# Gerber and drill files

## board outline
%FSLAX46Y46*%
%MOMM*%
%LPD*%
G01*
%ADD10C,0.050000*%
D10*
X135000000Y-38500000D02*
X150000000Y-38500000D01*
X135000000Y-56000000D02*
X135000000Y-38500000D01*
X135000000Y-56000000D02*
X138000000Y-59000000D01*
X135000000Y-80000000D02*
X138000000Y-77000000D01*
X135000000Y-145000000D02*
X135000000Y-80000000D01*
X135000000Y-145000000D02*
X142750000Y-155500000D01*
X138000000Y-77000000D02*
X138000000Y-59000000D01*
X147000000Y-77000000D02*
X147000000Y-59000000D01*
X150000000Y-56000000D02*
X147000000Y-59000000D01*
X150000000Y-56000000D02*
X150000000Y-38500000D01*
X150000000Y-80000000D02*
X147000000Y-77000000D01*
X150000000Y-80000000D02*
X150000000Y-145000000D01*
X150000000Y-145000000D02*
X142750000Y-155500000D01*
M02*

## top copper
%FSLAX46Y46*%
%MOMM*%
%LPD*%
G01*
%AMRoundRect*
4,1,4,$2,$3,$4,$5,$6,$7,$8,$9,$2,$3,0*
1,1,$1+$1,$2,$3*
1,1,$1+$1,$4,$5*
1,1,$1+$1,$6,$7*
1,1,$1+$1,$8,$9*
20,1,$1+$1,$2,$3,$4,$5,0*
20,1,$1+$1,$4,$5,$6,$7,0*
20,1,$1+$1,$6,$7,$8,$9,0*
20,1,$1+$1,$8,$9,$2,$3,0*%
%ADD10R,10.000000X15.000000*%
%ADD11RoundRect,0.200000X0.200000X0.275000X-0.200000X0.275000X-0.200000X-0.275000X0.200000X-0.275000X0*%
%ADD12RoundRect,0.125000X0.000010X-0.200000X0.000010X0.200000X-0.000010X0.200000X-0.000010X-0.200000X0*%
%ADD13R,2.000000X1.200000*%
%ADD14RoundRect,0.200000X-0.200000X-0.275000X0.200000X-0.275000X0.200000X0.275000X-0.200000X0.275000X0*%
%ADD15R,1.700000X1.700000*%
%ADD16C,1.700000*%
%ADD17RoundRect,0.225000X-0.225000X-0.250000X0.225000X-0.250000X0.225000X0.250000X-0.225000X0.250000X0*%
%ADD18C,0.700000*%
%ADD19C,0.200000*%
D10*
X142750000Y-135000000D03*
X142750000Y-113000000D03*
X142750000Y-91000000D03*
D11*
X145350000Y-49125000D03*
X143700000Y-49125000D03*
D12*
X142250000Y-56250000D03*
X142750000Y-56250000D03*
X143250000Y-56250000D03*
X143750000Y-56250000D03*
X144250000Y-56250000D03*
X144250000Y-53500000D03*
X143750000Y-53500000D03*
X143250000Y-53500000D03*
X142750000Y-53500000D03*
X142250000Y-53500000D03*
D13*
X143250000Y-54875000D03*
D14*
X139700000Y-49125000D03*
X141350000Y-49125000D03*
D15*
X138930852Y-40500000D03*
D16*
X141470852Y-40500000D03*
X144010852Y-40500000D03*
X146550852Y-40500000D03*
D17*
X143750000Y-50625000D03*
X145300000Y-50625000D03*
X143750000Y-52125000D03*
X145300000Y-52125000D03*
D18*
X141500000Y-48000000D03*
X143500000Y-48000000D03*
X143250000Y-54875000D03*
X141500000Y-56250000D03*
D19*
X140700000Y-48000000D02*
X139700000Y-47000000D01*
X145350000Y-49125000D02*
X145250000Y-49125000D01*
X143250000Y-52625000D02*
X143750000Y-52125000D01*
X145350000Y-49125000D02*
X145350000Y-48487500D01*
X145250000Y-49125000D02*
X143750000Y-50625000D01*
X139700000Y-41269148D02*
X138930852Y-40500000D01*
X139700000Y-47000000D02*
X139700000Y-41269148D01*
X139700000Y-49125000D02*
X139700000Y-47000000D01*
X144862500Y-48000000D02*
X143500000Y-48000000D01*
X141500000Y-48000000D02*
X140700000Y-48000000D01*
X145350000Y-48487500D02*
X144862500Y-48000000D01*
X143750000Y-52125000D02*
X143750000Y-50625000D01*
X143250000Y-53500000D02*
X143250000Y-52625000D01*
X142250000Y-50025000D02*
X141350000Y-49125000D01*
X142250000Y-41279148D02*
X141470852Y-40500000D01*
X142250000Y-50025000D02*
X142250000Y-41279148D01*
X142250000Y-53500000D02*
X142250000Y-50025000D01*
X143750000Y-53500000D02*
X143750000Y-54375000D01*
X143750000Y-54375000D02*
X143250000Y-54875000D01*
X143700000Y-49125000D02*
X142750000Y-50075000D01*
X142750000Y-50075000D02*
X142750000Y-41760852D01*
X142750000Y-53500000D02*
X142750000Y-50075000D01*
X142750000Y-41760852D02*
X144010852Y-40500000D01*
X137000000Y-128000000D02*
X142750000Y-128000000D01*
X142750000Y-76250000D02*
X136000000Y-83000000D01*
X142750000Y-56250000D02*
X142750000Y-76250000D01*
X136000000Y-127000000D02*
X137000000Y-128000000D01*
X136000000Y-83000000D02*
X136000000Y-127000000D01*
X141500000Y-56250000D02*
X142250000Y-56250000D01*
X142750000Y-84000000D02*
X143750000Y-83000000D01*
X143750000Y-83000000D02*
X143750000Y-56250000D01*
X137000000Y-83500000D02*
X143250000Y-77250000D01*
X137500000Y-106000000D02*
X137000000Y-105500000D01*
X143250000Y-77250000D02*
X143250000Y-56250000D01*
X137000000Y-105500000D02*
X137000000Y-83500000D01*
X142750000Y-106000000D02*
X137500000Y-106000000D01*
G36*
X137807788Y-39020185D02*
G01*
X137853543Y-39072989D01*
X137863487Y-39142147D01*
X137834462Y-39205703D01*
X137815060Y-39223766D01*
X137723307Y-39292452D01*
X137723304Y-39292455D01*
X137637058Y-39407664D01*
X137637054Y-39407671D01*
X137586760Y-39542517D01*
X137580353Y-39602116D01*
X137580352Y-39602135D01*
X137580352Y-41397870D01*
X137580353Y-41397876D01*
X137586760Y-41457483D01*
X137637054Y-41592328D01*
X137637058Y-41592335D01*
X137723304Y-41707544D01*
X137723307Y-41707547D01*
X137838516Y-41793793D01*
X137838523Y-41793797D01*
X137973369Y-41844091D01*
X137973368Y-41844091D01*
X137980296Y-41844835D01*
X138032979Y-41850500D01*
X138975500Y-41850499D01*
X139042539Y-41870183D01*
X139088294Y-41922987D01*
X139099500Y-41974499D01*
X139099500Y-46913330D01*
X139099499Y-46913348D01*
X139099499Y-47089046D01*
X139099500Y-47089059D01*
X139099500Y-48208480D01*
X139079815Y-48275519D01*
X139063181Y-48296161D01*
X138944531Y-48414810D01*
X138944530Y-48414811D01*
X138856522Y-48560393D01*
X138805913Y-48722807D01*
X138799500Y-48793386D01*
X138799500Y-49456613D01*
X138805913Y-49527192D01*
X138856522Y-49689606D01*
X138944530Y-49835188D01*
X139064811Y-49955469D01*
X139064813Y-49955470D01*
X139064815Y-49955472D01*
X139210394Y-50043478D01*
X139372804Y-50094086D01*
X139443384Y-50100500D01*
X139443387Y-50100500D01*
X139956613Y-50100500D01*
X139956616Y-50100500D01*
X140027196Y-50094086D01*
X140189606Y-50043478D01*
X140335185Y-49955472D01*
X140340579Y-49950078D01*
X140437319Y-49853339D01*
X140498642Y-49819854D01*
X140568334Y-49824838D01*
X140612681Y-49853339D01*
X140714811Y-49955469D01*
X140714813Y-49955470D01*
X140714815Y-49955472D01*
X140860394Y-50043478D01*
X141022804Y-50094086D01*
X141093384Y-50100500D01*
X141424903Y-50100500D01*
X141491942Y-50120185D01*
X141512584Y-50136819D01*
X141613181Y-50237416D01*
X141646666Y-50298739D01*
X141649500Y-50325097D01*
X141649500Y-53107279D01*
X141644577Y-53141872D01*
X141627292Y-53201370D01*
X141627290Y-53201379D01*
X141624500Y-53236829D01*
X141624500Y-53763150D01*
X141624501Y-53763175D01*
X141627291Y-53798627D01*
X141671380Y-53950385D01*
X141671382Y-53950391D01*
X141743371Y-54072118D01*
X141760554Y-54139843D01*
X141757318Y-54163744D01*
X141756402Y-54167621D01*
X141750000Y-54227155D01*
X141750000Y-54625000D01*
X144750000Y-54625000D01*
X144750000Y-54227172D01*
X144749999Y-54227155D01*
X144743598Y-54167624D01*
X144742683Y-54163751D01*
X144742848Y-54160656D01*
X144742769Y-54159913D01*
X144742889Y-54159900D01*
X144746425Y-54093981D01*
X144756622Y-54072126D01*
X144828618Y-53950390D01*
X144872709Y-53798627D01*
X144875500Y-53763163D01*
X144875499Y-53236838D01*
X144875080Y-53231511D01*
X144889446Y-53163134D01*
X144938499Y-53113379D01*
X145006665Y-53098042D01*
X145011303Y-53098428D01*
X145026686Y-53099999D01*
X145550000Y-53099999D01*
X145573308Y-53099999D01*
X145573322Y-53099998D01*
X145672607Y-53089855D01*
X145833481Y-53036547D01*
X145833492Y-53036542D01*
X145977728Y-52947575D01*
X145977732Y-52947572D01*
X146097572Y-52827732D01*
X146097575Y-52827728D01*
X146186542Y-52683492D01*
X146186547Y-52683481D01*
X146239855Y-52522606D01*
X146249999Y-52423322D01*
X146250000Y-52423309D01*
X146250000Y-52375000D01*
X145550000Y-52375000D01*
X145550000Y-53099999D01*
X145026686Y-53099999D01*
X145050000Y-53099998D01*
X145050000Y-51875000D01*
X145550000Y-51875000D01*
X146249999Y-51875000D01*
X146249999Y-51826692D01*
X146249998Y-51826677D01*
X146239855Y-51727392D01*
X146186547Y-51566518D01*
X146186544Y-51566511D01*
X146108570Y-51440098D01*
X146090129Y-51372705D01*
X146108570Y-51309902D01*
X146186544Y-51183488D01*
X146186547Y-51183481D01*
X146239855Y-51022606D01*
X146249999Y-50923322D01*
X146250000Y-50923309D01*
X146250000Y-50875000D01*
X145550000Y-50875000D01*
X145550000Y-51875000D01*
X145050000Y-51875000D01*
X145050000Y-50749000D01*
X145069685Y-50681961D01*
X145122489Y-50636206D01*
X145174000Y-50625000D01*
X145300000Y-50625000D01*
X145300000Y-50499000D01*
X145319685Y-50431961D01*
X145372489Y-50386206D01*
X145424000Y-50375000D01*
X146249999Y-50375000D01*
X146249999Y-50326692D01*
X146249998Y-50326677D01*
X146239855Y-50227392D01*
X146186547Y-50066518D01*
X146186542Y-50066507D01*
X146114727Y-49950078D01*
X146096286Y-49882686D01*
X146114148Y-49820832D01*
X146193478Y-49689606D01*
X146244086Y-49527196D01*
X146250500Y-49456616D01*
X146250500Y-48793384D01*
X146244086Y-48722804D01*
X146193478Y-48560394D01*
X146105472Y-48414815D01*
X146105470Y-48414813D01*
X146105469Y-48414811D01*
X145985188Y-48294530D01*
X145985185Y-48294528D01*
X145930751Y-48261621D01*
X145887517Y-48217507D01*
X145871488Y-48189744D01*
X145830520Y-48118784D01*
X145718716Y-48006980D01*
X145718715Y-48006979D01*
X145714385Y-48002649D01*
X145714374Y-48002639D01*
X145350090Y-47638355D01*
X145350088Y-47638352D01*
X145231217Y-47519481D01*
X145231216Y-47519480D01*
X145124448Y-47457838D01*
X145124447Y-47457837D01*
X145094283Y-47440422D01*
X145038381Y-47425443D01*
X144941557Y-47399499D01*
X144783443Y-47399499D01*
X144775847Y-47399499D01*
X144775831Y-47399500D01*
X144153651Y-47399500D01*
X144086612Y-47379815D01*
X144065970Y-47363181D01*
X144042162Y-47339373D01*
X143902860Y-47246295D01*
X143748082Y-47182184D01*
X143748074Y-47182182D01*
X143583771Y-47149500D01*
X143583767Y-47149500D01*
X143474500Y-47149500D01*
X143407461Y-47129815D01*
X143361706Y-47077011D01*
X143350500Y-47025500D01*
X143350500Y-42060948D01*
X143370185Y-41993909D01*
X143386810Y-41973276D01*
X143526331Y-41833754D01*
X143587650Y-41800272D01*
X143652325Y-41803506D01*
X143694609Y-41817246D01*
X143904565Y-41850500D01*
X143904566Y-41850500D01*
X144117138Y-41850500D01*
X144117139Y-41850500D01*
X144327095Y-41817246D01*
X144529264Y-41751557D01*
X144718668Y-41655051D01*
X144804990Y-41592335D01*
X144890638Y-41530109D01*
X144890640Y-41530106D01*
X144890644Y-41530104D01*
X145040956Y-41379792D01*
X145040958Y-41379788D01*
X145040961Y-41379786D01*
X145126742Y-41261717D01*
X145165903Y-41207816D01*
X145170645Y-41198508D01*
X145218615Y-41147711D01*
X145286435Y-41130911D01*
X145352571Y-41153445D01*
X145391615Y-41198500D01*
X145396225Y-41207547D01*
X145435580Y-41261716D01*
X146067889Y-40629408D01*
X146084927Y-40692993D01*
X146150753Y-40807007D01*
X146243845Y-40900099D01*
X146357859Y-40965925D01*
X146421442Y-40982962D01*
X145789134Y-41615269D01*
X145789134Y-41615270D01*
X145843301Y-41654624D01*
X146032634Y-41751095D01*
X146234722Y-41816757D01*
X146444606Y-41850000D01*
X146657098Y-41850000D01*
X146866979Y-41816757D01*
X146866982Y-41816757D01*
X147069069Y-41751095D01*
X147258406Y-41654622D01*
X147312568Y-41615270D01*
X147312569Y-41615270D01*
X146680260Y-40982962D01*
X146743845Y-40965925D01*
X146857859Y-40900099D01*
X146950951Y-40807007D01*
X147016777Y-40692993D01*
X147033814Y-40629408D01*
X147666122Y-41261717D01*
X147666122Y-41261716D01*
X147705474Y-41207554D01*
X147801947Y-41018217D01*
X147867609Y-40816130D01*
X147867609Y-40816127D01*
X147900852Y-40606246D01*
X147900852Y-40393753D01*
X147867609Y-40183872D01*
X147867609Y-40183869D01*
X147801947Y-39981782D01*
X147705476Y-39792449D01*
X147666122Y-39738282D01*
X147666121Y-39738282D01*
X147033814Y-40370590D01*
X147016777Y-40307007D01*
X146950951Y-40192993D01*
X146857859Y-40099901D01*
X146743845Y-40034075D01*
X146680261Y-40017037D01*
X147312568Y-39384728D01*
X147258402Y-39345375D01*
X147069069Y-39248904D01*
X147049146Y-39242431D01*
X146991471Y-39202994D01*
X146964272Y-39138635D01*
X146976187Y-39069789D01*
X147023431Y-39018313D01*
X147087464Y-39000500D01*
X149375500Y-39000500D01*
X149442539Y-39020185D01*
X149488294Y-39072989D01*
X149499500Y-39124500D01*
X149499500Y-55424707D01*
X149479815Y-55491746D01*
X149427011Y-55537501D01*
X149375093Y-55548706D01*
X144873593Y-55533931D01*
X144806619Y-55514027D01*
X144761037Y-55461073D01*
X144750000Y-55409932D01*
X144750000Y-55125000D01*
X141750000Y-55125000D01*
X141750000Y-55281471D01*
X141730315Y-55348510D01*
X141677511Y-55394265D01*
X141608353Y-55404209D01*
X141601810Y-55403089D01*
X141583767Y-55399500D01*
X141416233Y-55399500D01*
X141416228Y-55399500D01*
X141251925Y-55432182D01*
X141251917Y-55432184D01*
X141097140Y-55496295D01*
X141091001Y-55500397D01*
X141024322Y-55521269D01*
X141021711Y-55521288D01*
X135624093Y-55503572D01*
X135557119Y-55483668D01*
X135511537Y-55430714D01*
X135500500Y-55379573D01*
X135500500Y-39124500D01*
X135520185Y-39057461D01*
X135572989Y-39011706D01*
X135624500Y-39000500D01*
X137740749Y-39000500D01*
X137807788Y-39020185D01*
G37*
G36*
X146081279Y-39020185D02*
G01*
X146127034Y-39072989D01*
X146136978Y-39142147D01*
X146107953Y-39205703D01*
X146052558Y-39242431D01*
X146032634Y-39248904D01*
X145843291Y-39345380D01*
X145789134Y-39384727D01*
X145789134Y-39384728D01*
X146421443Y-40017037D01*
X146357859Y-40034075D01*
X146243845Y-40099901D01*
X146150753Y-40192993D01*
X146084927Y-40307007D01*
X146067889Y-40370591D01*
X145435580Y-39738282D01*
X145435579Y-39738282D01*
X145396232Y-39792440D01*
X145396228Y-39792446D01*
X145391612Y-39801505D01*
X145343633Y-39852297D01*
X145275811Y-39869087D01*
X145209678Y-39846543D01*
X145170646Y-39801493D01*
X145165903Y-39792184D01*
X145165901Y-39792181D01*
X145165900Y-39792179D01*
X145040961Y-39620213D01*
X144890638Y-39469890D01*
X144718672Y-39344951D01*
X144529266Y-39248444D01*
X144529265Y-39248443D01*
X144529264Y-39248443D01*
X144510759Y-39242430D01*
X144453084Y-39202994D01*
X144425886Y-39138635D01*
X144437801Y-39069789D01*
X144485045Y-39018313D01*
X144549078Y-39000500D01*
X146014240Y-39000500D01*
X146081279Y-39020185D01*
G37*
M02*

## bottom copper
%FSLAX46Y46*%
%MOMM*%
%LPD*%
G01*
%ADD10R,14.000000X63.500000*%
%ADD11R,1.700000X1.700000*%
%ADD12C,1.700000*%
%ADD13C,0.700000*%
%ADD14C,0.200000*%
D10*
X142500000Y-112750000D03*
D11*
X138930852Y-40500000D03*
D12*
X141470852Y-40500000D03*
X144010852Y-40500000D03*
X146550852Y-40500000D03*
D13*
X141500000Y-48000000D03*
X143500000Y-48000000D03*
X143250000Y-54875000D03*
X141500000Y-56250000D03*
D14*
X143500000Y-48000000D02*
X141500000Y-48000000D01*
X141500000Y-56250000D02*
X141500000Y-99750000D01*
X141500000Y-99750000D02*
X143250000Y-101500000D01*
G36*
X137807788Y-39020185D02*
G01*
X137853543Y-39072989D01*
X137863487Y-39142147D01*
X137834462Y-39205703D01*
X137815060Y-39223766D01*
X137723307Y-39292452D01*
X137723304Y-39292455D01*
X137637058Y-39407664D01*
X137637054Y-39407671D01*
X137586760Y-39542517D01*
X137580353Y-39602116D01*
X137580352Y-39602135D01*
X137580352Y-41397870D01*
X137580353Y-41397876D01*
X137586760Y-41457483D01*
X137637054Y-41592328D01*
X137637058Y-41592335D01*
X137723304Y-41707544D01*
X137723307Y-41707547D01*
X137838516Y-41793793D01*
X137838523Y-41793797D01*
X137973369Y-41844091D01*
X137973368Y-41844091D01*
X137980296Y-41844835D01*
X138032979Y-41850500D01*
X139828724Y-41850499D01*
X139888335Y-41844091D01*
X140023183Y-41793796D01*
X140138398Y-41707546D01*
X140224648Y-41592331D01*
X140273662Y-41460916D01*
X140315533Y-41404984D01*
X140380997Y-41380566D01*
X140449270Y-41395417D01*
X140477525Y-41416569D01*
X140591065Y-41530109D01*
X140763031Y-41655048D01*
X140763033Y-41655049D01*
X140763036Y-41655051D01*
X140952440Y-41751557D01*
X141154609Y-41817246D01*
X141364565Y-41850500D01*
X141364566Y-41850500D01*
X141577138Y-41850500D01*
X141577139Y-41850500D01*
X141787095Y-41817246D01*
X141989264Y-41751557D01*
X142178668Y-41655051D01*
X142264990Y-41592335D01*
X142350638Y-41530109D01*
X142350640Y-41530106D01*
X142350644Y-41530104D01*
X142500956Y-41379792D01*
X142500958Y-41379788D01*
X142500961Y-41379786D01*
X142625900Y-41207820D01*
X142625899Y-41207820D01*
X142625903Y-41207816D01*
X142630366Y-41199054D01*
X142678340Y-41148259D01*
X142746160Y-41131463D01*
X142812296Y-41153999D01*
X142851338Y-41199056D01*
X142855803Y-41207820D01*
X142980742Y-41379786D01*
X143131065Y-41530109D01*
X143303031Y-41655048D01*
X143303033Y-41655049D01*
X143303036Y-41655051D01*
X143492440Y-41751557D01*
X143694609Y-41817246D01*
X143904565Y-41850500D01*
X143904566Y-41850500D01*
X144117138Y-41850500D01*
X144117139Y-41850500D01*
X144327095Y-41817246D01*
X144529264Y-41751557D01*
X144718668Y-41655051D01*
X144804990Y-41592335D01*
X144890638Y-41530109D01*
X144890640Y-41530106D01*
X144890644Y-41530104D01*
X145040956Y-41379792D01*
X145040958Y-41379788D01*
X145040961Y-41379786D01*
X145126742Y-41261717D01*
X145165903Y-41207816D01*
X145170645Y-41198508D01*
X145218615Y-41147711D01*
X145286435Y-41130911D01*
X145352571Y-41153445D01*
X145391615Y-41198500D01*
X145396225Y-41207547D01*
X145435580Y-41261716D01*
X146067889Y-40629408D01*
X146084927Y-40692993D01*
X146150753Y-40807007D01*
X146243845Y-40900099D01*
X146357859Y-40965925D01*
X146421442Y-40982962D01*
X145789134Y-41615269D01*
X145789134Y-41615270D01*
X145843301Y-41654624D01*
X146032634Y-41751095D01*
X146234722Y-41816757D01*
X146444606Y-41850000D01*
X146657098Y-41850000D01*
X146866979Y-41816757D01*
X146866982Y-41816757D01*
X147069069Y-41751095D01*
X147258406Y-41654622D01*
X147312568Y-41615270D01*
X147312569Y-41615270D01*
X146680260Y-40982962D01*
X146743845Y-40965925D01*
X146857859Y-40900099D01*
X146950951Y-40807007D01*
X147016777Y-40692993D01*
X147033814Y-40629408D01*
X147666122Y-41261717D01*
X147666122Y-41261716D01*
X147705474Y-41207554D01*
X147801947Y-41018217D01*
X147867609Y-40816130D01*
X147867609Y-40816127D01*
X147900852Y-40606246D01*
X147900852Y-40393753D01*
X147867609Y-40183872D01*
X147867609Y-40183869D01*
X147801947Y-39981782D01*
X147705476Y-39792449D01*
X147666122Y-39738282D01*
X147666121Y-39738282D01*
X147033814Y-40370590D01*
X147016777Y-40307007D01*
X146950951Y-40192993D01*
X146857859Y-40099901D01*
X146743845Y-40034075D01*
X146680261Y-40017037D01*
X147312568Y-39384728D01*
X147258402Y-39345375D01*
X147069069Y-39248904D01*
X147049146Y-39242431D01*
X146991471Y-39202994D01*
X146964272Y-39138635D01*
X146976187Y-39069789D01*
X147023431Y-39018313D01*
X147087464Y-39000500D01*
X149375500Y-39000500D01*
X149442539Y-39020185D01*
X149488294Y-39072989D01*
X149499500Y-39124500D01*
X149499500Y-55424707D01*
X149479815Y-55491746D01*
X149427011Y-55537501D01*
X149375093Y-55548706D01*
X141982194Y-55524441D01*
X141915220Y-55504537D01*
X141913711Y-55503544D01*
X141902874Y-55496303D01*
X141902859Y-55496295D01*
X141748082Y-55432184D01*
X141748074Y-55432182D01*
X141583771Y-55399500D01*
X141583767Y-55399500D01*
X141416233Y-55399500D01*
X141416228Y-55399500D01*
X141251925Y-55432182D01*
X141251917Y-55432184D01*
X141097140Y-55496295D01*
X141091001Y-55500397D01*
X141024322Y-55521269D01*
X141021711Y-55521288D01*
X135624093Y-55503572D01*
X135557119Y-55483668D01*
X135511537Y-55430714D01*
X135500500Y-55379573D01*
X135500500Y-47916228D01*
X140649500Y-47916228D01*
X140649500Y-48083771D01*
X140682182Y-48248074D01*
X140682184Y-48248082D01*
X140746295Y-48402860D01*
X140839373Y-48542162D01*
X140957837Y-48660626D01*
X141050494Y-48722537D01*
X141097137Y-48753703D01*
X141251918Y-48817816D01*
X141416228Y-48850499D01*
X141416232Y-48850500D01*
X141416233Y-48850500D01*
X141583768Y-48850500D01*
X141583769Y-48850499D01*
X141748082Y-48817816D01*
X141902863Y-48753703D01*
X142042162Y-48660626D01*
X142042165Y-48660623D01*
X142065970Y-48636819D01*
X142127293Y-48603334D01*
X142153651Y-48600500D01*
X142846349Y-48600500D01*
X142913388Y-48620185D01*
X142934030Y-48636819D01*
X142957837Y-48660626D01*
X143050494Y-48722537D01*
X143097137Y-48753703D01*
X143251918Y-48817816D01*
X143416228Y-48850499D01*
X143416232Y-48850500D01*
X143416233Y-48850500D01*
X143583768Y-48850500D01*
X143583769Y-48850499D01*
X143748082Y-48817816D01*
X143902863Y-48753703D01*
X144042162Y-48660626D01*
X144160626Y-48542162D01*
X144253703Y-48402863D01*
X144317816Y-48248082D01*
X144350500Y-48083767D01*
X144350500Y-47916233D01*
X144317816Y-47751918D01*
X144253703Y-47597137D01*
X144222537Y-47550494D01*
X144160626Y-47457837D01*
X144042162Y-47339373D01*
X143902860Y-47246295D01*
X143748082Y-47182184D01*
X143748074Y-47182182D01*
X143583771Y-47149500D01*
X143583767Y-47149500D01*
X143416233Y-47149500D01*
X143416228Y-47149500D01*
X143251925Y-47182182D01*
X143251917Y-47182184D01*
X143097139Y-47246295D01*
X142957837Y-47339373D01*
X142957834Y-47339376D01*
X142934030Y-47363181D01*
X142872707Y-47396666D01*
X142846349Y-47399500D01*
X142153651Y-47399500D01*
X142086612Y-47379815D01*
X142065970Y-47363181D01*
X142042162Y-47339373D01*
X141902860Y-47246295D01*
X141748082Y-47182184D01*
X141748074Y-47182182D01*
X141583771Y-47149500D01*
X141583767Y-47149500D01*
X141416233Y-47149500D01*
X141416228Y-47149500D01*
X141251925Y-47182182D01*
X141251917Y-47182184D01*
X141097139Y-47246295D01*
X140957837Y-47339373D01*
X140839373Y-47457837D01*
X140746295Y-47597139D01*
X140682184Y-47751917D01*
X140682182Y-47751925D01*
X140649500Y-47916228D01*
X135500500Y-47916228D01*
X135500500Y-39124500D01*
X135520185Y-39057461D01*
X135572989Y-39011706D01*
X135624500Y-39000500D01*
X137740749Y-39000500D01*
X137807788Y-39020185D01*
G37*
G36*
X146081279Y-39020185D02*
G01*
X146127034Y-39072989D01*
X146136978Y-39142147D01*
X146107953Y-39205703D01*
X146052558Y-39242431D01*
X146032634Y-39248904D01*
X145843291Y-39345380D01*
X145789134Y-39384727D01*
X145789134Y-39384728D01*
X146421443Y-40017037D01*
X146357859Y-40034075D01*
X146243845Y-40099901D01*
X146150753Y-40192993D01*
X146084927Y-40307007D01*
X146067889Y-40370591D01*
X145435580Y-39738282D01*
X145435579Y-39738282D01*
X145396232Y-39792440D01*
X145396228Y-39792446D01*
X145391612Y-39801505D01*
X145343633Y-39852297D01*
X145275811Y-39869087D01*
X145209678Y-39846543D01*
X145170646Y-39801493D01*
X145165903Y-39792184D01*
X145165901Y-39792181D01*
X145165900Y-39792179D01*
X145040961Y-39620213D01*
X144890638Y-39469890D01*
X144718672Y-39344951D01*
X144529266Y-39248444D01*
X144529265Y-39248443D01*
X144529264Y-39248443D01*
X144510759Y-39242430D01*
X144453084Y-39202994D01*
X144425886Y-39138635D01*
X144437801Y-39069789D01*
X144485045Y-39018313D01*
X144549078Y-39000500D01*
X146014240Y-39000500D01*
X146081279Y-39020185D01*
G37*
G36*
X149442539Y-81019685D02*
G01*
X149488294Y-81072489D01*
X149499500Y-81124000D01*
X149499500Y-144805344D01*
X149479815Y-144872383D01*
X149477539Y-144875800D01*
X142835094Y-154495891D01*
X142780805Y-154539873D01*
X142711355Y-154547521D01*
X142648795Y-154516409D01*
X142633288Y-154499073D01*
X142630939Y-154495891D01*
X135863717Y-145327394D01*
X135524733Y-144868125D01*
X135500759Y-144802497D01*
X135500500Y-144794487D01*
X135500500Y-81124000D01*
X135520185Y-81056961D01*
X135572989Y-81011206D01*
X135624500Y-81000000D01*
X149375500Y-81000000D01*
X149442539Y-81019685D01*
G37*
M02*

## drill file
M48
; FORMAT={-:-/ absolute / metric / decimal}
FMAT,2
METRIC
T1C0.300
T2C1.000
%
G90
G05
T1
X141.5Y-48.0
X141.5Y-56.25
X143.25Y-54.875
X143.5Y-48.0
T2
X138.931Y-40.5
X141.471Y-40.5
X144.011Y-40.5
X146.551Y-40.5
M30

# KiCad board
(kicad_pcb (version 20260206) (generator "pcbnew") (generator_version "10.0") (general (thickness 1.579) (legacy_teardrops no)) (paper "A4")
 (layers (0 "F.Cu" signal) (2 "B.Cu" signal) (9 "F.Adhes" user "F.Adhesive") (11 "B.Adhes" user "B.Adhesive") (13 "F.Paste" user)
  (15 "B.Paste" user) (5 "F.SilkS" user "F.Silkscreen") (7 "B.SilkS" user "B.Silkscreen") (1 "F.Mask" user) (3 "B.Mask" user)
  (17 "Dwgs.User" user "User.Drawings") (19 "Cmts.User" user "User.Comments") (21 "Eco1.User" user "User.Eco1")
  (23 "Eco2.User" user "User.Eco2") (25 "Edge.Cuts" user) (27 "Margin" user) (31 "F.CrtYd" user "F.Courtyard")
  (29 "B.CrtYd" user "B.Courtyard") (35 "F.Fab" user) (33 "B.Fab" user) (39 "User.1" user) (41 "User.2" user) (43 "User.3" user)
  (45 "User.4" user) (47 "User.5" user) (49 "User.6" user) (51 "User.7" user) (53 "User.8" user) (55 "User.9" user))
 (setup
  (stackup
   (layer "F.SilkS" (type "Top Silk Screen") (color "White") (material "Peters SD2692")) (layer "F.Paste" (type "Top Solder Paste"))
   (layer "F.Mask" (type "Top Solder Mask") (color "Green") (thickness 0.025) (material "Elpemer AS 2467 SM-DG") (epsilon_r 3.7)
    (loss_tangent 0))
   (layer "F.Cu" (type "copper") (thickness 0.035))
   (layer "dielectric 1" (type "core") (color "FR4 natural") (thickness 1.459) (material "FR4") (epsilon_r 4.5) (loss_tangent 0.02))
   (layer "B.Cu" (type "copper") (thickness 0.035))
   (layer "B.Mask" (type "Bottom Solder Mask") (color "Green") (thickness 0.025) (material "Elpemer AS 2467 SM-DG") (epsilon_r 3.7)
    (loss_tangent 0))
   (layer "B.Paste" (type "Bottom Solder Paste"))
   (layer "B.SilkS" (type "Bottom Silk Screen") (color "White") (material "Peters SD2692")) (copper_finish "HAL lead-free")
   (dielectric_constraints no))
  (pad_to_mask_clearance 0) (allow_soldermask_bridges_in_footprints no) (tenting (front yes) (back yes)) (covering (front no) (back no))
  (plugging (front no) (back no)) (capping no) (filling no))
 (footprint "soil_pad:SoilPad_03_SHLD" (layer "F.Cu") (at 142.75 102)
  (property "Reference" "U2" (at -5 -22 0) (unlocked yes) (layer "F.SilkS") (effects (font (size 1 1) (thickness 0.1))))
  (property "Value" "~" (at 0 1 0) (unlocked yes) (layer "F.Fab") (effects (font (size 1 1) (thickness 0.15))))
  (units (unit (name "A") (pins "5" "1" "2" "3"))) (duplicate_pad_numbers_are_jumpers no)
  (pad "1" smd rect (at 0 26) (size 10 15) (drill (offset 0 7)) (layers "F.Cu") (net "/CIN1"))
  (pad "2" smd rect (at 0 4) (size 10 15) (drill (offset 0 7)) (layers "F.Cu") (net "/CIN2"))
  (pad "3" smd rect (at 0 -18) (size 10 15) (drill (offset 0 7)) (layers "F.Cu") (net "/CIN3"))
  (pad "5" smd rect (at -0.25 10.75) (size 14 63.5) (layers "B.Cu") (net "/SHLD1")))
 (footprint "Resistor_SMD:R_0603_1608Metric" (layer "F.Cu") (at 144.525 49.125 180)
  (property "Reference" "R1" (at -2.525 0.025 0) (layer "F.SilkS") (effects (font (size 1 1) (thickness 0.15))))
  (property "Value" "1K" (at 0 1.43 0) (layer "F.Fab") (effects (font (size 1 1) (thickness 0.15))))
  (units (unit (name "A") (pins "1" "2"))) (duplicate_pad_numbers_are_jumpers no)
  (pad "1" smd roundrect (at -0.825 0 180) (size 0.8 0.95) (layers "F.Cu" "F.Mask" "F.Paste") (roundrect_rratio 0.25) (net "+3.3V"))
  (pad "2" smd roundrect (at 0.825 0 180) (size 0.8 0.95) (layers "F.Cu" "F.Mask" "F.Paste") (roundrect_rratio 0.25) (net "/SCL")))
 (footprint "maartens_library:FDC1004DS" (layer "F.Cu") (at 143.25 54.875 90)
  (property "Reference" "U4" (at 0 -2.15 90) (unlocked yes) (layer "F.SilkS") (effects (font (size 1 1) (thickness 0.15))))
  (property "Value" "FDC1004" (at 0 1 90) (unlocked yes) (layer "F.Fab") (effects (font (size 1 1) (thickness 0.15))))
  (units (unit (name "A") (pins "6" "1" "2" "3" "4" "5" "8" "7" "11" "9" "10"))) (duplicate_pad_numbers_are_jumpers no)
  (pad "1" smd roundrect (at -1.375 -1 90) (size 0.65 0.25) (layers "F.Cu" "F.Mask" "F.Paste") (roundrect_rratio 0.5) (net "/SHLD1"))
  (pad "2" smd roundrect (at -1.375 -0.5 90) (size 0.65 0.25) (layers "F.Cu" "F.Mask" "F.Paste") (roundrect_rratio 0.5) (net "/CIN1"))
  (pad "3" smd roundrect (at -1.375 0 90) (size 0.65 0.25) (layers "F.Cu" "F.Mask" "F.Paste") (roundrect_rratio 0.5) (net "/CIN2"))
  (pad "4" smd roundrect (at -1.375 0.5 90) (size 0.65 0.25) (layers "F.Cu" "F.Mask" "F.Paste") (roundrect_rratio 0.5) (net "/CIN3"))
  (pad "5" smd roundrect (at -1.375 1 90) (size 0.65 0.25) (layers "F.Cu" "F.Mask" "F.Paste") (roundrect_rratio 0.5)
   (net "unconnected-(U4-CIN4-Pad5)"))
  (pad "6" smd roundrect (at 1.375 1 90) (size 0.65 0.25) (layers "F.Cu" "F.Mask" "F.Paste") (roundrect_rratio 0.5)
   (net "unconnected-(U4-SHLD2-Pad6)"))
  (pad "7" smd roundrect (at 1.375 0.5 90) (size 0.65 0.25) (layers "F.Cu" "F.Mask" "F.Paste") (roundrect_rratio 0.5) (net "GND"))
  (pad "8" smd roundrect (at 1.375 0 90) (size 0.65 0.25) (layers "F.Cu" "F.Mask" "F.Paste") (roundrect_rratio 0.5) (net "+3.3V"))
  (pad "9" smd roundrect (at 1.375 -0.5 90) (size 0.65 0.25) (layers "F.Cu" "F.Mask" "F.Paste") (roundrect_rratio 0.5) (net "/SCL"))
  (pad "10" smd roundrect (at 1.375 -1 90) (size 0.65 0.25) (layers "F.Cu" "F.Mask" "F.Paste") (roundrect_rratio 0.5) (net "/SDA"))
  (pad "11" smd rect (at 0 0 90) (size 1.2 2) (layers "F.Cu" "F.Mask" "F.Paste") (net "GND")))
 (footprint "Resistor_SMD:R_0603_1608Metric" (layer "F.Cu") (at 140.525 49.125)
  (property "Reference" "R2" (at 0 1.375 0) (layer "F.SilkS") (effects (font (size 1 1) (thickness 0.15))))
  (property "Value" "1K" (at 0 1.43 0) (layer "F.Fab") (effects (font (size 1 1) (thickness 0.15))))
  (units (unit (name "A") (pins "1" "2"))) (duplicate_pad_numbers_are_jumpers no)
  (pad "1" smd roundrect (at -0.825 0) (size 0.8 0.95) (layers "F.Cu" "F.Mask" "F.Paste") (roundrect_rratio 0.25) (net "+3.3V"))
  (pad "2" smd roundrect (at 0.825 0) (size 0.8 0.95) (layers "F.Cu" "F.Mask" "F.Paste") (roundrect_rratio 0.25) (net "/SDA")))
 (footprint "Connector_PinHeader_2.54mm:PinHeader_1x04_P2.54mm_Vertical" (layer "F.Cu") (at 138.930852 40.5 90)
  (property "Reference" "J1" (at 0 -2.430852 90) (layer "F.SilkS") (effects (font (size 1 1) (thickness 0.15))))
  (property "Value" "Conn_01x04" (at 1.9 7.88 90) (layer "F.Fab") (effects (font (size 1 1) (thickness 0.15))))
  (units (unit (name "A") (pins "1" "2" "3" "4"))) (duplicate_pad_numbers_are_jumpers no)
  (pad "1" thru_hole rect (at 0 0 90) (size 1.7 1.7) (drill 1) (layers "*.Cu" "*.Mask") (remove_unused_layers no) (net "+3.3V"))
  (pad "2" thru_hole circle (at 0 2.54 90) (size 1.7 1.7) (drill 1) (layers "*.Cu" "*.Mask") (remove_unused_layers no) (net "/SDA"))
  (pad "3" thru_hole circle (at 0 5.08 90) (size 1.7 1.7) (drill 1) (layers "*.Cu" "*.Mask") (remove_unused_layers no) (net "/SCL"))
  (pad "4" thru_hole circle (at 0 7.62 90) (size 1.7 1.7) (drill 1) (layers "*.Cu" "*.Mask") (remove_unused_layers no) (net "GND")))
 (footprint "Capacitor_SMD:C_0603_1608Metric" (layer "F.Cu") (at 144.525 50.625)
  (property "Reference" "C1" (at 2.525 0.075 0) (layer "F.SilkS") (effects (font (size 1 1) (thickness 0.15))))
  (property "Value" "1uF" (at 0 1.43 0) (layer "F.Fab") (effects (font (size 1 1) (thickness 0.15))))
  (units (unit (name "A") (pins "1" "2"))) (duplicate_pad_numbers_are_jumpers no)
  (pad "1" smd roundrect (at -0.775 0) (size 0.9 0.95) (layers "F.Cu" "F.Mask" "F.Paste") (roundrect_rratio 0.25) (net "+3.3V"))
  (pad "2" smd roundrect (at 0.775 0) (size 0.9 0.95) (layers "F.Cu" "F.Mask" "F.Paste") (roundrect_rratio 0.25) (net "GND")))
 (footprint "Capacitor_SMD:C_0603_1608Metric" (layer "F.Cu") (at 144.525 52.125)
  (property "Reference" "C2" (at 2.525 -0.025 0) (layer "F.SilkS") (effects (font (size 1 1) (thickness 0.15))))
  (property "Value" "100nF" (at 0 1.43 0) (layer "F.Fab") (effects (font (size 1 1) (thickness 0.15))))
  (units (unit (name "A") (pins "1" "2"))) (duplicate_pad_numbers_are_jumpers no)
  (pad "1" smd roundrect (at -0.775 0) (size 0.9 0.95) (layers "F.Cu" "F.Mask" "F.Paste") (roundrect_rratio 0.25) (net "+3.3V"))
  (pad "2" smd roundrect (at 0.775 0) (size 0.9 0.95) (layers "F.Cu" "F.Mask" "F.Paste") (roundrect_rratio 0.25) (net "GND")))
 (gr_line (start 135 38.5) (end 150 38.5) (stroke (width 0.05) (type default)) (layer "Edge.Cuts"))
 (gr_line (start 135 56) (end 135 38.5) (stroke (width 0.05) (type default)) (layer "Edge.Cuts"))
 (gr_line (start 135 56) (end 138 59) (stroke (width 0.05) (type default)) (layer "Edge.Cuts"))
 (gr_line (start 135 80) (end 138 77) (stroke (width 0.05) (type default)) (layer "Edge.Cuts"))
 (gr_line (start 135 145) (end 135 80) (stroke (width 0.05) (type default)) (layer "Edge.Cuts"))
 (gr_line (start 135 145) (end 142.75 155.5) (stroke (width 0.05) (type default)) (layer "Edge.Cuts"))
 (gr_line (start 138 77) (end 138 59) (stroke (width 0.05) (type default)) (layer "Edge.Cuts"))
 (gr_line (start 147 77) (end 147 59) (stroke (width 0.05) (type default)) (layer "Edge.Cuts"))
 (gr_line (start 150 56) (end 147 59) (stroke (width 0.05) (type default)) (layer "Edge.Cuts"))
 (gr_line (start 150 56) (end 150 38.5) (stroke (width 0.05) (type default)) (layer "Edge.Cuts"))
 (gr_line (start 150 80) (end 147 77) (stroke (width 0.05) (type default)) (layer "Edge.Cuts"))
 (gr_line (start 150 80) (end 150 145) (stroke (width 0.05) (type default)) (layer "Edge.Cuts"))
 (gr_line (start 150 145) (end 142.75 155.5) (stroke (width 0.05) (type default)) (layer "Edge.Cuts"))
 (segment (start 140.7 48) (end 139.7 47) (width 0.2) (layer "F.Cu") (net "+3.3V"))
 (segment (start 145.35 49.125) (end 145.25 49.125) (width 0.2) (layer "F.Cu") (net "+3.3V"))
 (segment (start 143.25 52.625) (end 143.75 52.125) (width 0.2) (layer "F.Cu") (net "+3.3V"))
 (segment (start 145.35 49.125) (end 145.35 48.4875) (width 0.2) (layer "F.Cu") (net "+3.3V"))
 (segment (start 145.25 49.125) (end 143.75 50.625) (width 0.2) (layer "F.Cu") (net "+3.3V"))
 (segment (start 139.7 41.269148) (end 138.930852 40.5) (width 0.2) (layer "F.Cu") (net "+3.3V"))
 (segment (start 139.7 47) (end 139.7 41.269148) (width 0.2) (layer "F.Cu") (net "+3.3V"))
 (segment (start 139.7 49.125) (end 139.7 47) (width 0.2) (layer "F.Cu") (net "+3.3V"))
 (segment (start 144.8625 48) (end 143.5 48) (width 0.2) (layer "F.Cu") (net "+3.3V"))
 (segment (start 141.5 48) (end 140.7 48) (width 0.2) (layer "F.Cu") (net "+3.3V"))
 (segment (start 145.35 48.4875) (end 144.8625 48) (width 0.2) (layer "F.Cu") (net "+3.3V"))
 (segment (start 143.75 52.125) (end 143.75 50.625) (width 0.2) (layer "F.Cu") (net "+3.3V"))
 (segment (start 143.25 53.5) (end 143.25 52.625) (width 0.2) (layer "F.Cu") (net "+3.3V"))
 (via (at 141.5 48) (size 0.7) (drill 0.3) (layers "F.Cu" "B.Cu") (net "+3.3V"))
 (via (at 143.5 48) (size 0.7) (drill 0.3) (layers "F.Cu" "B.Cu") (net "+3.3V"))
 (segment (start 143.5 48) (end 141.5 48) (width 0.2) (layer "B.Cu") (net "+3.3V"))
 (segment (start 142.25 50.025) (end 141.35 49.125) (width 0.2) (layer "F.Cu") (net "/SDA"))
 (segment (start 142.25 41.279148) (end 141.470852 40.5) (width 0.2) (layer "F.Cu") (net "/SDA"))
 (segment (start 142.25 50.025) (end 142.25 41.279148) (width 0.2) (layer "F.Cu") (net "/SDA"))
 (segment (start 142.25 53.5) (end 142.25 50.025) (width 0.2) (layer "F.Cu") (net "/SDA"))
 (segment (start 143.75 53.5) (end 143.75 54.375) (width 0.2) (layer "F.Cu") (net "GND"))
 (segment (start 143.75 54.375) (end 143.25 54.875) (width 0.2) (layer "F.Cu") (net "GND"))
 (via (at 143.25 54.875) (size 0.7) (drill 0.3) (layers "F.Cu" "B.Cu") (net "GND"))
 (segment (start 143.7 49.125) (end 142.75 50.075) (width 0.2) (layer "F.Cu") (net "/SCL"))
 (segment (start 142.75 50.075) (end 142.75 41.760852) (width 0.2) (layer "F.Cu") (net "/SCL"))
 (segment (start 142.75 53.5) (end 142.75 50.075) (width 0.2) (layer "F.Cu") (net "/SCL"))
 (segment (start 142.75 41.760852) (end 144.010852 40.5) (width 0.2) (layer "F.Cu") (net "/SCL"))
 (segment (start 137 128) (end 142.75 128) (width 0.2) (layer "F.Cu") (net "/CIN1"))
 (segment (start 142.75 76.25) (end 136 83) (width 0.2) (layer "F.Cu") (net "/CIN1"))
 (segment (start 142.75 56.25) (end 142.75 76.25) (width 0.2) (layer "F.Cu") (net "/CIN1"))
 (segment (start 136 127) (end 137 128) (width 0.2) (layer "F.Cu") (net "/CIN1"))
 (segment (start 136 83) (end 136 127) (width 0.2) (layer "F.Cu") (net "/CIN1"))
 (segment (start 141.5 56.25) (end 142.25 56.25) (width 0.2) (layer "F.Cu") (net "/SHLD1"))
 (via (at 141.5 56.25) (size 0.7) (drill 0.3) (layers "F.Cu" "B.Cu") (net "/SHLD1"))
 (segment (start 141.5 56.25) (end 141.5 99.75) (width 0.2) (layer "B.Cu") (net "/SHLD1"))
 (segment (start 141.5 99.75) (end 143.25 101.5) (width 0.2) (layer "B.Cu") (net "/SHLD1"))
 (segment (start 142.75 84) (end 143.75 83) (width 0.2) (layer "F.Cu") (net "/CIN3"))
 (segment (start 143.75 83) (end 143.75 56.25) (width 0.2) (layer "F.Cu") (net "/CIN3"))
 (segment (start 137 83.5) (end 143.25 77.25) (width 0.2) (layer "F.Cu") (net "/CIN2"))
 (segment (start 137.5 106) (end 137 105.5) (width 0.2) (layer "F.Cu") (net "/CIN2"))
 (segment (start 143.25 77.25) (end 143.25 56.25) (width 0.2) (layer "F.Cu") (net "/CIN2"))
 (segment (start 137 105.5) (end 137 83.5) (width 0.2) (layer "F.Cu") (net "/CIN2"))
 (segment (start 142.75 106) (end 137.5 106) (width 0.2) (layer "F.Cu") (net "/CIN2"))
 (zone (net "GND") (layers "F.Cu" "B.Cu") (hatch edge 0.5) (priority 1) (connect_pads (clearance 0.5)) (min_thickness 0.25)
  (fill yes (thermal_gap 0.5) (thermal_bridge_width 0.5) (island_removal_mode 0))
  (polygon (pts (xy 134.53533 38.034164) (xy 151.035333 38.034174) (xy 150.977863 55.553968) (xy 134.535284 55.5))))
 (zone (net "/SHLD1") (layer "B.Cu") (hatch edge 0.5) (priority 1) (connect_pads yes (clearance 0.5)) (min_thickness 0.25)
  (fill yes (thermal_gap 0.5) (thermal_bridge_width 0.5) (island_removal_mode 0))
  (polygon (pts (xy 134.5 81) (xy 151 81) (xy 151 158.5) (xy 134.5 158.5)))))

